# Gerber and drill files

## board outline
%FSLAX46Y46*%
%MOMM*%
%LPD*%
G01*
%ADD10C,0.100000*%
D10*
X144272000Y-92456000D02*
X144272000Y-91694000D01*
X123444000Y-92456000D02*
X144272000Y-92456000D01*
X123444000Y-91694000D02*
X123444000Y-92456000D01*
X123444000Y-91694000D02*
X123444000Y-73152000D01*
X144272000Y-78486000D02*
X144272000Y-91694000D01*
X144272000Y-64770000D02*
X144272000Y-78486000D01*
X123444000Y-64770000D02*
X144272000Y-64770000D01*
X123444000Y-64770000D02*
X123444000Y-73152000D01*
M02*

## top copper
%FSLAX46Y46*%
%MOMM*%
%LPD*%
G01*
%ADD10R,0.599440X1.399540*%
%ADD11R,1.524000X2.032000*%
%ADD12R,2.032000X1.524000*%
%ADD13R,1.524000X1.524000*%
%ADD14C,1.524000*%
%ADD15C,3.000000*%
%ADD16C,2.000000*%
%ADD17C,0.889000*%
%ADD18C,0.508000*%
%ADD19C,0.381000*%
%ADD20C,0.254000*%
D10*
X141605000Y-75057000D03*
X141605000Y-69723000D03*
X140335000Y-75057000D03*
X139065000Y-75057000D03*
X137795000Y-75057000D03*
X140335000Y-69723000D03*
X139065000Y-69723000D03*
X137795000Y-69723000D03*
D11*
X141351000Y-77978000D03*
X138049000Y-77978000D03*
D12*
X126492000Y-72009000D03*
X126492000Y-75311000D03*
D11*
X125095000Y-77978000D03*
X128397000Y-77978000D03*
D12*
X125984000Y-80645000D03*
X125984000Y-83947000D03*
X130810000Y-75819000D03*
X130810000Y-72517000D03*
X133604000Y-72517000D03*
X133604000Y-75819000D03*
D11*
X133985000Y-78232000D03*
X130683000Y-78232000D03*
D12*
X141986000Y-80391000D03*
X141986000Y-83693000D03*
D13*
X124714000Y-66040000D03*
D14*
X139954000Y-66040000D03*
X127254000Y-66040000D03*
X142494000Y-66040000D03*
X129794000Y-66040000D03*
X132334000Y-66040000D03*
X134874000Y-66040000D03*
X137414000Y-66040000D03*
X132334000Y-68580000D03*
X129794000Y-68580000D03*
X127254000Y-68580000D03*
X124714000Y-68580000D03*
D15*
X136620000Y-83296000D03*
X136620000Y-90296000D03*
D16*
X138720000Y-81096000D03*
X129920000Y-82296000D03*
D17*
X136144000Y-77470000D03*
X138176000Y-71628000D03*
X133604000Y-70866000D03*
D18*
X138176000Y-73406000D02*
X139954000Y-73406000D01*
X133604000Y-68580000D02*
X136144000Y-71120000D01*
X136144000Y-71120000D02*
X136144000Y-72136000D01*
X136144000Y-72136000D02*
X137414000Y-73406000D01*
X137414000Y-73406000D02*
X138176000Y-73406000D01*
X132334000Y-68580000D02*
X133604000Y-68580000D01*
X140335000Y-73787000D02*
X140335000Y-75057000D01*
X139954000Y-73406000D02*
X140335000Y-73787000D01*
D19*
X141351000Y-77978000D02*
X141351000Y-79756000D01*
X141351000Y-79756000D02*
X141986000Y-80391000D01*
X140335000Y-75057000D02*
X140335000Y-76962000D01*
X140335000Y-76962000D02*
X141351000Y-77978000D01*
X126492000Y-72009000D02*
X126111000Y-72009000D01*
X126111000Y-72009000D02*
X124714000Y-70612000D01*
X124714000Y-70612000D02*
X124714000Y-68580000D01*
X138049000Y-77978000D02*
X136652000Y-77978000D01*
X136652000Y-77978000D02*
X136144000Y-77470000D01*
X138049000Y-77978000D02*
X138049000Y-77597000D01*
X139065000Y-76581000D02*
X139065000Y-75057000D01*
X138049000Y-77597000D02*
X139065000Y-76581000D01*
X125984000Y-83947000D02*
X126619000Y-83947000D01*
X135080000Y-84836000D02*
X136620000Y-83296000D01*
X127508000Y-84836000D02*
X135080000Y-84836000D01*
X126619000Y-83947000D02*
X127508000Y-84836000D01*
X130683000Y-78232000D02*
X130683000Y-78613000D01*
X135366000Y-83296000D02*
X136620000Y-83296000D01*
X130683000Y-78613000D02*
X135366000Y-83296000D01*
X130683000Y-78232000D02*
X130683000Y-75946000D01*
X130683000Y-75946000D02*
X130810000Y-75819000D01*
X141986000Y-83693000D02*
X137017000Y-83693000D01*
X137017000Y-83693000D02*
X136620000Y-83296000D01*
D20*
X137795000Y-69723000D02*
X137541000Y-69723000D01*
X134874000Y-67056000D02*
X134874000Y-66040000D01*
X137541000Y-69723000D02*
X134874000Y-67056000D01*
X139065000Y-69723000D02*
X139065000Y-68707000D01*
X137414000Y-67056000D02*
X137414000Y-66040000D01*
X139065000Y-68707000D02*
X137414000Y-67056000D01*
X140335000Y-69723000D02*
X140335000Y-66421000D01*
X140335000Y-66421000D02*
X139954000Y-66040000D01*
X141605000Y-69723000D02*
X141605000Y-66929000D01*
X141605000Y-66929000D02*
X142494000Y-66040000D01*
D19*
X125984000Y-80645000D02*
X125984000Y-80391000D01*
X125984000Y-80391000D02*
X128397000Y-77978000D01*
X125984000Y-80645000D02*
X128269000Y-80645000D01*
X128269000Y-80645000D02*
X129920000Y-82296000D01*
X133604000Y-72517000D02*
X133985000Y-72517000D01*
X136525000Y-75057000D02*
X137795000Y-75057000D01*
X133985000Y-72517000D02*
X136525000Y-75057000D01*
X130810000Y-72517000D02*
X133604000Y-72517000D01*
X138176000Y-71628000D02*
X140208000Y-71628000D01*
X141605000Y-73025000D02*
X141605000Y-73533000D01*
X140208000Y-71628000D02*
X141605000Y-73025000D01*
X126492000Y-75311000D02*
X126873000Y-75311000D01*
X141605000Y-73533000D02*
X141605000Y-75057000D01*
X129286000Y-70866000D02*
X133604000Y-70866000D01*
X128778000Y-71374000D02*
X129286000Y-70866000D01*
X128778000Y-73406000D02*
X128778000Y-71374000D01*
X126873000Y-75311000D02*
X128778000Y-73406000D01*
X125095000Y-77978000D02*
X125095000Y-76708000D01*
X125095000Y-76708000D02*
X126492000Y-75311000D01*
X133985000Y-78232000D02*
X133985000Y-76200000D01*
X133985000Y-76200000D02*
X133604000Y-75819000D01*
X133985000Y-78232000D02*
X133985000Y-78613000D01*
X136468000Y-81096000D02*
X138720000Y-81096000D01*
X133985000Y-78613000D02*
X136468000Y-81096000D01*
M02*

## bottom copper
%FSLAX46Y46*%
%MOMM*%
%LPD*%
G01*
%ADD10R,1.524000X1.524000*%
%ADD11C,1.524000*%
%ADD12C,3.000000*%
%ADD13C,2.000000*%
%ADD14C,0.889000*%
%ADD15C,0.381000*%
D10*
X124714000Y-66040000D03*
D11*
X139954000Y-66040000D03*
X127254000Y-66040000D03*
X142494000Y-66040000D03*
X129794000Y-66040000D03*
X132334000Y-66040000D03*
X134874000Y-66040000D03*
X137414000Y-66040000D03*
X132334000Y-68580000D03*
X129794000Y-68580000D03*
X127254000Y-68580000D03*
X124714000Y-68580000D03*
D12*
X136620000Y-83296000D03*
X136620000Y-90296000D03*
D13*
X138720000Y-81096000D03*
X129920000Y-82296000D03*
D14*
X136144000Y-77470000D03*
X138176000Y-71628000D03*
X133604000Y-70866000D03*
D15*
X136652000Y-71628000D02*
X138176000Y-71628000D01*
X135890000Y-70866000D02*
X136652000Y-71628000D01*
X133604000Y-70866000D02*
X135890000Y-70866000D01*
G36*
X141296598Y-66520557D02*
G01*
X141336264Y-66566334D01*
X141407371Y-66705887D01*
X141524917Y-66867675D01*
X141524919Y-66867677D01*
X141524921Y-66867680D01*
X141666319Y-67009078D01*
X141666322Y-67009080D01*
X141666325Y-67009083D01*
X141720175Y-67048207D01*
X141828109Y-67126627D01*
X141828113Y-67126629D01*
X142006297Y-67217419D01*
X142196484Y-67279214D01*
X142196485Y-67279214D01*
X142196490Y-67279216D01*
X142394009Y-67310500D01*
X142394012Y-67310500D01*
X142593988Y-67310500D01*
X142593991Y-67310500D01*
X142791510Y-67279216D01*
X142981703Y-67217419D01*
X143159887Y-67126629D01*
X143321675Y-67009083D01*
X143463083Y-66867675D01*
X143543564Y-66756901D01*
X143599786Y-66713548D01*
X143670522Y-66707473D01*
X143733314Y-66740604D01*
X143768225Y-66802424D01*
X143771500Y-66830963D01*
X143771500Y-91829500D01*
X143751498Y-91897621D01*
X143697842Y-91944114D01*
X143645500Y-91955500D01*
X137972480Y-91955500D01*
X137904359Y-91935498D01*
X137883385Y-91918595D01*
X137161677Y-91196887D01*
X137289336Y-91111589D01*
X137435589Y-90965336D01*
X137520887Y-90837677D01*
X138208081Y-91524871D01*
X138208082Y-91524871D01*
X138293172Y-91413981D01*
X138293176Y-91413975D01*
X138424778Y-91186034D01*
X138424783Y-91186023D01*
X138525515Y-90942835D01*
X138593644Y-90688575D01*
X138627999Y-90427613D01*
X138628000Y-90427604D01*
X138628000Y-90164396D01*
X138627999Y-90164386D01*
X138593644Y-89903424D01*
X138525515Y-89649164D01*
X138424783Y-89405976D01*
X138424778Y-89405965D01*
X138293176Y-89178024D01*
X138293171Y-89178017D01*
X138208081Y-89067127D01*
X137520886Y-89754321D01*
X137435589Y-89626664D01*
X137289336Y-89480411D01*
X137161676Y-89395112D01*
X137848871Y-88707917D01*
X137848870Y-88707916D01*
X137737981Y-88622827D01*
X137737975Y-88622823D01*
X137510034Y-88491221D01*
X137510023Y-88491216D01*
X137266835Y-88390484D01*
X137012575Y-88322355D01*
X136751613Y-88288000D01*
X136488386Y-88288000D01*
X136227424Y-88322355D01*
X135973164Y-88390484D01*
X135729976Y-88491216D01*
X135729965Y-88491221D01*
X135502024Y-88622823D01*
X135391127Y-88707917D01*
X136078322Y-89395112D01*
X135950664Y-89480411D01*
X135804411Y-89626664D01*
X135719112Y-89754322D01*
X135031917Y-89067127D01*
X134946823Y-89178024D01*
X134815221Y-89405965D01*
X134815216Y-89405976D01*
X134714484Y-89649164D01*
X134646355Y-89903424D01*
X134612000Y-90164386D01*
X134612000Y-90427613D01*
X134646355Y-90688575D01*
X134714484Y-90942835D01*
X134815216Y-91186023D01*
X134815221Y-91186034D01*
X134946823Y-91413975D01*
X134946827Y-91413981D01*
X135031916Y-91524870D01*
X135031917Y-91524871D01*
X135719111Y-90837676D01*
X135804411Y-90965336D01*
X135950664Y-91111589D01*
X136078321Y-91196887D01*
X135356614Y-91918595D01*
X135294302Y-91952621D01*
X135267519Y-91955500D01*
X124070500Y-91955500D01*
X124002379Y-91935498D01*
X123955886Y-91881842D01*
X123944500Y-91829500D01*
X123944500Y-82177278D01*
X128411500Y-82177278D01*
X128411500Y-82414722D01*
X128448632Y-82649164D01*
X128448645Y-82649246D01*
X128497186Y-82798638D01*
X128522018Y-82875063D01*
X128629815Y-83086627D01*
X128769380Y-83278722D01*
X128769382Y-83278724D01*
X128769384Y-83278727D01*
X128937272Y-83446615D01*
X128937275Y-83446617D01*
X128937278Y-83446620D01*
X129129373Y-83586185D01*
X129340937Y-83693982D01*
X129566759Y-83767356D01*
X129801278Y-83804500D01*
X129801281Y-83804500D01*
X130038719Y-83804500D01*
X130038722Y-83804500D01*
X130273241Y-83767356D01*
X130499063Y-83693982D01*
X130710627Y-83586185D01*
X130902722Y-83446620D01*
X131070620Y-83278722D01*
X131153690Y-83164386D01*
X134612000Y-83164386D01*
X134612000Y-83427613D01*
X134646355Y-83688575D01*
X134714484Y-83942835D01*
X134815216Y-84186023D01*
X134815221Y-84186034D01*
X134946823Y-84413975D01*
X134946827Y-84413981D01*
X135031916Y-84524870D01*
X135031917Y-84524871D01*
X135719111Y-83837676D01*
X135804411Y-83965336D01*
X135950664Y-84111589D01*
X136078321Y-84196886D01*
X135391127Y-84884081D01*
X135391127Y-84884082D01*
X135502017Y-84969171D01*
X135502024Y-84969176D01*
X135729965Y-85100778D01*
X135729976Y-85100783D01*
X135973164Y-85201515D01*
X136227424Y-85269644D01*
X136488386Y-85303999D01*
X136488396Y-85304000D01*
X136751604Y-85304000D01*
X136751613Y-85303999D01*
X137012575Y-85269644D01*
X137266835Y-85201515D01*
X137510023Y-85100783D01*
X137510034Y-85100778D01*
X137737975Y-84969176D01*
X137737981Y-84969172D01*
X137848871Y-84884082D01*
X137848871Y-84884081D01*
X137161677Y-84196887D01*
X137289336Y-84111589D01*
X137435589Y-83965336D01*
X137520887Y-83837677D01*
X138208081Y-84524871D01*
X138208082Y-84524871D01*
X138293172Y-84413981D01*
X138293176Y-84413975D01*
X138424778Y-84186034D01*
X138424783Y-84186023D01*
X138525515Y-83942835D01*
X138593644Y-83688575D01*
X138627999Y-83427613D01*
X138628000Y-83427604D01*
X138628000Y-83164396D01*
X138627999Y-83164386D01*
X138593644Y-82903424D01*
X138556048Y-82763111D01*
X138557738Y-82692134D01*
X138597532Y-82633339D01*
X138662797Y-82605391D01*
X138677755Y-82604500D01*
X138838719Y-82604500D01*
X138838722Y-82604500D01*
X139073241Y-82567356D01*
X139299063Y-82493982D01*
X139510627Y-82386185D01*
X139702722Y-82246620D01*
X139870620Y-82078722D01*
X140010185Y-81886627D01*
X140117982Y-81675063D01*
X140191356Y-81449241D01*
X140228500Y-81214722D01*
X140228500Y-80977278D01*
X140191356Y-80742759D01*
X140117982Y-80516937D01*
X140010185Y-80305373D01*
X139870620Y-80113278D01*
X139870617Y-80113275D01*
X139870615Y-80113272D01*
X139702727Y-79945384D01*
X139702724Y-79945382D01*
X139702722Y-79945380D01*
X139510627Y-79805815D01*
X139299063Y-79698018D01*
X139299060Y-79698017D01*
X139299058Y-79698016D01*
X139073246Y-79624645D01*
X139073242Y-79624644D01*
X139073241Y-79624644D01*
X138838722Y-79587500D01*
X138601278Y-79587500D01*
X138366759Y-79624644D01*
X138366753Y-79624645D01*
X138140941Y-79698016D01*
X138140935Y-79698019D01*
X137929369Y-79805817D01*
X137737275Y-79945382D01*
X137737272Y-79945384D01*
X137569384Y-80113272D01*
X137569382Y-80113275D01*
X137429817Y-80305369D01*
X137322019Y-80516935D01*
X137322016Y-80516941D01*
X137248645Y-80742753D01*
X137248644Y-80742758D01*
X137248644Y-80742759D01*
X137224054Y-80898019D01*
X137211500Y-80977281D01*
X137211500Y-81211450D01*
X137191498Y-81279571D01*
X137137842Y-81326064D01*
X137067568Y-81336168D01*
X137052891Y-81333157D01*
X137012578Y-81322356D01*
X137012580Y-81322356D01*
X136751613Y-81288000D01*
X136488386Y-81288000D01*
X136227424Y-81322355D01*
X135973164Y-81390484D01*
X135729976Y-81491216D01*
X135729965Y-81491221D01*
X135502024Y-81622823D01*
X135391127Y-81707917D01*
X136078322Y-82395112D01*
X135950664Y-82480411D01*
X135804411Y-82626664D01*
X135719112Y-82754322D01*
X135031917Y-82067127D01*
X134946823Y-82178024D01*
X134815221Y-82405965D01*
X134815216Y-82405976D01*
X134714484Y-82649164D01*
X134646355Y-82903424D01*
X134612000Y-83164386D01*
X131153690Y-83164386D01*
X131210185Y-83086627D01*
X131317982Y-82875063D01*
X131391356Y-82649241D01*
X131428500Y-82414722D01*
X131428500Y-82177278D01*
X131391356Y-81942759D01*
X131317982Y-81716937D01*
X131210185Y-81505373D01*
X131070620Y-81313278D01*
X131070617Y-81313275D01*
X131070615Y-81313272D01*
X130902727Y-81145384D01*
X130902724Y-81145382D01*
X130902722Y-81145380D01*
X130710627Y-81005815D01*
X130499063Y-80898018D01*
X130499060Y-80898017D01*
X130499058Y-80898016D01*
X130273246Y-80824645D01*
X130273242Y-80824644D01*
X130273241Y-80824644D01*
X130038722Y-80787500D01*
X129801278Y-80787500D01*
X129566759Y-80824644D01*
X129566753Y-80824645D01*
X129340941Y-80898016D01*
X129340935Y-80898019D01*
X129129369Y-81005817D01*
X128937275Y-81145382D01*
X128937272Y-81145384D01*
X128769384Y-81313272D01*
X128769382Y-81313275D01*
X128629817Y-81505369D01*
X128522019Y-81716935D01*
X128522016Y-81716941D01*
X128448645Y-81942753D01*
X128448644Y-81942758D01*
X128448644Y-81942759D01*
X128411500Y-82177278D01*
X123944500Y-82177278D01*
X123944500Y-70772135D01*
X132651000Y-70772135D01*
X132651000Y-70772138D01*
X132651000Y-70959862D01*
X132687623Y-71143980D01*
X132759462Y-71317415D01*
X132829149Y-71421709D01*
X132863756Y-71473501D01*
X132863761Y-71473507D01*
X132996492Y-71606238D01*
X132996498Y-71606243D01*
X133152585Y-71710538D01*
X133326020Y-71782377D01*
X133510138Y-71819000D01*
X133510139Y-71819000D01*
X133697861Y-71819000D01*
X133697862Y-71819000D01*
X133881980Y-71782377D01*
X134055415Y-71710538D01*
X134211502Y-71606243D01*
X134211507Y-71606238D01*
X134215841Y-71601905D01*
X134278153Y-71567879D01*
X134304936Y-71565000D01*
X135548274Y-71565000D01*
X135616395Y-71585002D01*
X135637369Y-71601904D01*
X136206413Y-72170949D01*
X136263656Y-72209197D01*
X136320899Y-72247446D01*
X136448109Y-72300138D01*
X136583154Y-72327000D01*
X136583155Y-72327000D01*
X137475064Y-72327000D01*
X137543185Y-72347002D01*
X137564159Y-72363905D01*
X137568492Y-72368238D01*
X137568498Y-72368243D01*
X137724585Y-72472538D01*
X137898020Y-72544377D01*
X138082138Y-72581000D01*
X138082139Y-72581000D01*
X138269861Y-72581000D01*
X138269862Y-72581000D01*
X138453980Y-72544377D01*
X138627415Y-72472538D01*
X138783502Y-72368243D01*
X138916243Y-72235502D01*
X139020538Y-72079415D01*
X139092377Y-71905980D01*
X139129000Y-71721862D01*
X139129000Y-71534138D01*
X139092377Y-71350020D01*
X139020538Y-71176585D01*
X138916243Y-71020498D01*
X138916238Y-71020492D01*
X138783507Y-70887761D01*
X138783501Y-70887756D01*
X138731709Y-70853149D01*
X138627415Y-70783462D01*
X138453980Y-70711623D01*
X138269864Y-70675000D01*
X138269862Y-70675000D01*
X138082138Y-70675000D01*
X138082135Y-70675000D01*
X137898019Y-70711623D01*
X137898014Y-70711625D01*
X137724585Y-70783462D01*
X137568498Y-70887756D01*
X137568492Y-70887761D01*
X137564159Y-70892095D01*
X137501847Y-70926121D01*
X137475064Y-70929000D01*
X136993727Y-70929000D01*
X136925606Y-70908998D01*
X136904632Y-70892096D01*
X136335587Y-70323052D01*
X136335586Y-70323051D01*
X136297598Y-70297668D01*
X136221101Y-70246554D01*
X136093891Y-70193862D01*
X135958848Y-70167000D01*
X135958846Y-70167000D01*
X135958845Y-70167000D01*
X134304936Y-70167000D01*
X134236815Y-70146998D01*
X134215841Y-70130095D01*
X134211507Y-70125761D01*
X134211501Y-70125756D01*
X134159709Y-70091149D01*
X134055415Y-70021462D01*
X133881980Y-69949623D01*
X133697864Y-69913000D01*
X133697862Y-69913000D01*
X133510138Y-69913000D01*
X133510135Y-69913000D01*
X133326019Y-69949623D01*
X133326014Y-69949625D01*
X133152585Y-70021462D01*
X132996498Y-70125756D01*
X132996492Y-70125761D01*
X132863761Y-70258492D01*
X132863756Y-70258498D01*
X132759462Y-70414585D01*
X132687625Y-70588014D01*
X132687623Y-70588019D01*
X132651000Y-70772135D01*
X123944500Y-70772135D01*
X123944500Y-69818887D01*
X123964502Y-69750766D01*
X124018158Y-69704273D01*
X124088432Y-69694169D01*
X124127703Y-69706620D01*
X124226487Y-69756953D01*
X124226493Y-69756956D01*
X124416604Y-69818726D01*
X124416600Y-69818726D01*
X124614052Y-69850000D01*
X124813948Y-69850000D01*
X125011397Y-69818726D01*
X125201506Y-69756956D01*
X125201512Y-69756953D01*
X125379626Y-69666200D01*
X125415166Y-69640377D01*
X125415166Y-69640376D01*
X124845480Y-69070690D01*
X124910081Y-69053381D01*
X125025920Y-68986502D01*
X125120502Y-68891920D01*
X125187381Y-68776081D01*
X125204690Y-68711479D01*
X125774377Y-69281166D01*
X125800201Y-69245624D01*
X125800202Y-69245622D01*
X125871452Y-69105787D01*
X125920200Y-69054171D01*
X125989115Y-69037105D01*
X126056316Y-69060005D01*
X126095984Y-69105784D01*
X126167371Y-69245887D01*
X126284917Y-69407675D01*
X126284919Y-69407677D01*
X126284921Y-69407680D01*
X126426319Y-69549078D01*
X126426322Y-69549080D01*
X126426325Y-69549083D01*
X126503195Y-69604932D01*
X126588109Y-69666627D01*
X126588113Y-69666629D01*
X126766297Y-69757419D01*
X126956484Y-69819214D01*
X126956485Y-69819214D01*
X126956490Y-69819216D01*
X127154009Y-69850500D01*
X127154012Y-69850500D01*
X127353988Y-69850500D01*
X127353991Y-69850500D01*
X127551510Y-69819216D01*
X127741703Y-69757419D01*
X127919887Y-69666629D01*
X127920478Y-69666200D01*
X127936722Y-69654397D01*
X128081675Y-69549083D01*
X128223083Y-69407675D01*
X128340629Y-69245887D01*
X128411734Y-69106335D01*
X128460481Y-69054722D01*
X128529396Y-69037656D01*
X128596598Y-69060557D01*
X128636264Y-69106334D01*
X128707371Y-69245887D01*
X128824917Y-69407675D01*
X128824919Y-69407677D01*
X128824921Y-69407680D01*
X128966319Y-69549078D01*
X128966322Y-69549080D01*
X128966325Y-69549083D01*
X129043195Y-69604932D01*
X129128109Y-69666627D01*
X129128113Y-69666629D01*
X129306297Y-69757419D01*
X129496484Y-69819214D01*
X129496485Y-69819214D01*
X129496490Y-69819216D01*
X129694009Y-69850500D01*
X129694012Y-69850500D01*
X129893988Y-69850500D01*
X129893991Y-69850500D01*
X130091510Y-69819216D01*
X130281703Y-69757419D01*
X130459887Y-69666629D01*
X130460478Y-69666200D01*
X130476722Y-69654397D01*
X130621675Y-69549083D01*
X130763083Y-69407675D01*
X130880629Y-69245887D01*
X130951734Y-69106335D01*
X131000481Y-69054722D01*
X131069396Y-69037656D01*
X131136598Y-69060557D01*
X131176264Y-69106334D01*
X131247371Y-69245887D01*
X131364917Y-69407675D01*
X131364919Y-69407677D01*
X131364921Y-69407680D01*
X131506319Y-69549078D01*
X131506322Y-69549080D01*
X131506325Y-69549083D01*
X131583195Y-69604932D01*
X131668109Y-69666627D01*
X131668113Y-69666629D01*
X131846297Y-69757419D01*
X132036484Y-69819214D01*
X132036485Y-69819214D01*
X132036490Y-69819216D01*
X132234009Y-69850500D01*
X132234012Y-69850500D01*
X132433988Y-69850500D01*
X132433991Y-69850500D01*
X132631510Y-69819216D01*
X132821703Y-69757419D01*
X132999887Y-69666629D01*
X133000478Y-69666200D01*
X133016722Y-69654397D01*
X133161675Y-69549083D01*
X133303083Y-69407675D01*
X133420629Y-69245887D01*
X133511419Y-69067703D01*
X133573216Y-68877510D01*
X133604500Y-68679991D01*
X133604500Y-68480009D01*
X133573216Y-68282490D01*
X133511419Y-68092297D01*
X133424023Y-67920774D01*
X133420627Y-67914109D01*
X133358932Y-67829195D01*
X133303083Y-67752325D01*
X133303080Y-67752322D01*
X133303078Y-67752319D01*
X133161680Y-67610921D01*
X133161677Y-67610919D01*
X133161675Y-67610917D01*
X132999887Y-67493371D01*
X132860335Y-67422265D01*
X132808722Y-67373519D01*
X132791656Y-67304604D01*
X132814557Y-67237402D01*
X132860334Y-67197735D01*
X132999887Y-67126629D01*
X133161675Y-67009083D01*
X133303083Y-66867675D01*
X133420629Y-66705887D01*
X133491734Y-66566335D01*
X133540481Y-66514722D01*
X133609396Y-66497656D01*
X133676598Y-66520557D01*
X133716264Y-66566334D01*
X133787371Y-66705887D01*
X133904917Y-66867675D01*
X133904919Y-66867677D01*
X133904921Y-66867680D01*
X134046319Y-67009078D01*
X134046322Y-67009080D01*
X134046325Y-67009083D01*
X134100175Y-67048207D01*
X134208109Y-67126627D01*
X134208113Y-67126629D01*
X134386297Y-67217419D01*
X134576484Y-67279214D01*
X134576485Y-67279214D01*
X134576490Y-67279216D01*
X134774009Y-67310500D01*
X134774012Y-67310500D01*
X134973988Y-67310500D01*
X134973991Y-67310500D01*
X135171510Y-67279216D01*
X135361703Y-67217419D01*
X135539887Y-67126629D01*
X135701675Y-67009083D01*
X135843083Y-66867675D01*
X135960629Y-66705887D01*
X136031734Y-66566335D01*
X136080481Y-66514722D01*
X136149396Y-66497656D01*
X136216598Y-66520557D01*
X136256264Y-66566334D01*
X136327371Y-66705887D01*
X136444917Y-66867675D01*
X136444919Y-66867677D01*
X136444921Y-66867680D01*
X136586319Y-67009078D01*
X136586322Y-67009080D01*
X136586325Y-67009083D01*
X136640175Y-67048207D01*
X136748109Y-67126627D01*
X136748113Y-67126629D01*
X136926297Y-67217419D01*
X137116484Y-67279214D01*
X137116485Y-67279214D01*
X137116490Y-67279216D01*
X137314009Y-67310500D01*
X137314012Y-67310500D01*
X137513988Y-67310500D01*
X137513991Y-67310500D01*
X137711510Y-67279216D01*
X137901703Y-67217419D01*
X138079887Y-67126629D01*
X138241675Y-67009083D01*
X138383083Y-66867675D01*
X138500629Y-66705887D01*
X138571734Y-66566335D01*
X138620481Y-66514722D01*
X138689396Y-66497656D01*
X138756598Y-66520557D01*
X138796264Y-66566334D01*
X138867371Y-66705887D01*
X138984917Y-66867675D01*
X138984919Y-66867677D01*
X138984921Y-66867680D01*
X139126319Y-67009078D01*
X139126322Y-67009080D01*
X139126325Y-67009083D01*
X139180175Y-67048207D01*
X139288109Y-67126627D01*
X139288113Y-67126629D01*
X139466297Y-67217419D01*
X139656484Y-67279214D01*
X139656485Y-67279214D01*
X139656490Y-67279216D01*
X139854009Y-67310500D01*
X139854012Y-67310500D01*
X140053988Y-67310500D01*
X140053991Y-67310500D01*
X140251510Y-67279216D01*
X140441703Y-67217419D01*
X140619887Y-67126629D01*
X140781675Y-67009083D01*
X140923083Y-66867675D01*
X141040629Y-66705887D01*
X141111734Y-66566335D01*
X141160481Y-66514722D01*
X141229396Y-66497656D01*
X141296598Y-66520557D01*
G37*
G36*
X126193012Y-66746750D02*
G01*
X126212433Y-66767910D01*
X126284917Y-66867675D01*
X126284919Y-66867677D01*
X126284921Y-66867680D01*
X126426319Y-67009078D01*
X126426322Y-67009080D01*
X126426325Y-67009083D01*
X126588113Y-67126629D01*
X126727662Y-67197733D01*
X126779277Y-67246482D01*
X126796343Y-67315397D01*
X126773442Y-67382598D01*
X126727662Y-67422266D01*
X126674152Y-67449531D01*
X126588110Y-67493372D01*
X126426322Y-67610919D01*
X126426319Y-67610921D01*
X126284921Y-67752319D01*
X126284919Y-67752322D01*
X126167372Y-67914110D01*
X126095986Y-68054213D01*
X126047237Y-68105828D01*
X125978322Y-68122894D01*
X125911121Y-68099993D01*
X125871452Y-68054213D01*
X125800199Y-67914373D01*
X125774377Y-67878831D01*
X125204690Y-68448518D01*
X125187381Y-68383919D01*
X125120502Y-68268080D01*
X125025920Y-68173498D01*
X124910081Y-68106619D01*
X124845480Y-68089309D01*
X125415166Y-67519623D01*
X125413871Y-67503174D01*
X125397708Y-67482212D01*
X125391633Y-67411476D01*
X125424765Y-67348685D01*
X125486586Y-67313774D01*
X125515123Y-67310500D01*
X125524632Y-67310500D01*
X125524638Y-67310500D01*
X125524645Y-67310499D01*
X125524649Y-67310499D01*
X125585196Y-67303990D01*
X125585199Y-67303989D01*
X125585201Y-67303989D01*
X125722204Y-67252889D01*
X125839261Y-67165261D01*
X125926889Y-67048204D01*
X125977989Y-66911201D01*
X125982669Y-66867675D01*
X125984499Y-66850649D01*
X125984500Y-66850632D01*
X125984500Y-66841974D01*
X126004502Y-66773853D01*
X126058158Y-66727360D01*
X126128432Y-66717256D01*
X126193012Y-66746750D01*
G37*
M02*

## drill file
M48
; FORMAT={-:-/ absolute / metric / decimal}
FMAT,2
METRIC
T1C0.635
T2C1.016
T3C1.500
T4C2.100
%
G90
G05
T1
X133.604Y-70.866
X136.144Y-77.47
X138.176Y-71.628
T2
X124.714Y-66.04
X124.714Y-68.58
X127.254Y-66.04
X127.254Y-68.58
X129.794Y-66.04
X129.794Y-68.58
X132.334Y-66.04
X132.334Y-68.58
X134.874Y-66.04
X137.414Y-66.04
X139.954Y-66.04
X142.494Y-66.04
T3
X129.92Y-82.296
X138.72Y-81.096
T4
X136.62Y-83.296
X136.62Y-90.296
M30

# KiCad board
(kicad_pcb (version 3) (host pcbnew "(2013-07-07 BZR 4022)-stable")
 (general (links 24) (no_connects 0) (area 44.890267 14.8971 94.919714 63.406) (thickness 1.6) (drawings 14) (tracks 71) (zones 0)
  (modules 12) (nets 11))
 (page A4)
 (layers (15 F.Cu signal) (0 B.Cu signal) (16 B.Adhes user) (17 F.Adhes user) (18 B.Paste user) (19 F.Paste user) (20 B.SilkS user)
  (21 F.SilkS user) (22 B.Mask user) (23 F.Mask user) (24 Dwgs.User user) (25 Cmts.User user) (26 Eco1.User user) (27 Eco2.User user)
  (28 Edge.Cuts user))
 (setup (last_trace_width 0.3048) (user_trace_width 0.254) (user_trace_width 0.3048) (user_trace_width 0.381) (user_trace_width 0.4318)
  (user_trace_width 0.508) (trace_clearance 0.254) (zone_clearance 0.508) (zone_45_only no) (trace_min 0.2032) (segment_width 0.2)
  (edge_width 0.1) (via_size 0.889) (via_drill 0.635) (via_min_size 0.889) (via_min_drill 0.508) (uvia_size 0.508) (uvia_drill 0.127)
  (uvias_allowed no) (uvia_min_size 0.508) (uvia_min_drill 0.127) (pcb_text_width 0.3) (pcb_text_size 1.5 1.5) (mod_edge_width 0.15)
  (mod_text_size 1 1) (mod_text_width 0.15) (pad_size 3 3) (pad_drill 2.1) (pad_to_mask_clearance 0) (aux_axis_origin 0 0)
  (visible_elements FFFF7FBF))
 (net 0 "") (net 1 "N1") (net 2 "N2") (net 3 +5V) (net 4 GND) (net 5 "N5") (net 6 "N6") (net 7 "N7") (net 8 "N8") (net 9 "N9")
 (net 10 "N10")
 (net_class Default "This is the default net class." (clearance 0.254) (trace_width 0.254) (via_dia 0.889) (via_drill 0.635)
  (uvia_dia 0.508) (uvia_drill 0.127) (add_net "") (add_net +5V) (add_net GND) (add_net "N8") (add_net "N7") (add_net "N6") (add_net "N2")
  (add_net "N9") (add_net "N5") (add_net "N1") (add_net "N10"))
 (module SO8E (layer F.Cu) (at 139.7 72.39 180)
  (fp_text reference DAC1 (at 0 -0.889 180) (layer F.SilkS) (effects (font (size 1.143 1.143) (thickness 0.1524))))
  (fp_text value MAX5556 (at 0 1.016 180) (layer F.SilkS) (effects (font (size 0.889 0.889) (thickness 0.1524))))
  (pad 8 smd rect (at -1.905 -2.667 180) (size 0.59944 1.39954) (layers F.Cu F.Paste F.Mask) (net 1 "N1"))
  (pad 1 smd rect (at -1.905 2.667 180) (size 0.59944 1.39954) (layers F.Cu F.Paste F.Mask) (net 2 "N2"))
  (pad 7 smd rect (at -0.635 -2.667 180) (size 0.59944 1.39954) (layers F.Cu F.Paste F.Mask) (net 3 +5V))
  (pad 6 smd rect (at 0.635 -2.667 180) (size 0.59944 1.39954) (layers F.Cu F.Paste F.Mask) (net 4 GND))
  (pad 5 smd rect (at 1.905 -2.667 180) (size 0.59944 1.39954) (layers F.Cu F.Paste F.Mask) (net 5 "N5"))
  (pad 2 smd rect (at -0.635 2.667 180) (size 0.59944 1.39954) (layers F.Cu F.Paste F.Mask) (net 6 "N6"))
  (pad 3 smd rect (at 0.635 2.667 180) (size 0.59944 1.39954) (layers F.Cu F.Paste F.Mask) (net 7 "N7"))
  (pad 4 smd rect (at 1.905 2.667 180) (size 0.59944 1.39954) (layers F.Cu F.Paste F.Mask) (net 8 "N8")))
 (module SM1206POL (layer F.Cu) (at 139.7 77.978 180)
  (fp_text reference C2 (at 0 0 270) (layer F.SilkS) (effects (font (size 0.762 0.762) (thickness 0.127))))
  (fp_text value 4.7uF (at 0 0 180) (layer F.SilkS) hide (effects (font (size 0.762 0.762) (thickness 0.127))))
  (pad 1 smd rect (at -1.651 0 180) (size 1.524 2.032) (layers F.Cu F.Paste F.Mask) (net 3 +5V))
  (pad 2 smd rect (at 1.651 0 180) (size 1.524 2.032) (layers F.Cu F.Paste F.Mask) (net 4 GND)))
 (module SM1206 (layer F.Cu) (at 126.492 73.66 270)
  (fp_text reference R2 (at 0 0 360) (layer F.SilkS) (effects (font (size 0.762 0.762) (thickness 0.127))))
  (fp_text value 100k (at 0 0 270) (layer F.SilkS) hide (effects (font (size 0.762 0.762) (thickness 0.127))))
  (pad 1 smd rect (at -1.651 0 270) (size 1.524 2.032) (layers F.Cu F.Paste F.Mask) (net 4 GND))
  (pad 2 smd rect (at 1.651 0 270) (size 1.524 2.032) (layers F.Cu F.Paste F.Mask) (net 1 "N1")))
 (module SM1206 (layer F.Cu) (at 126.746 77.978)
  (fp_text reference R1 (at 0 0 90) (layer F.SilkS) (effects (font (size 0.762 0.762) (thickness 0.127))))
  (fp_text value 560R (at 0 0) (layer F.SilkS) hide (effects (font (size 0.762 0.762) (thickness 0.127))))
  (pad 1 smd rect (at -1.651 0) (size 1.524 2.032) (layers F.Cu F.Paste F.Mask) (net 1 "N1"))
  (pad 2 smd rect (at 1.651 0) (size 1.524 2.032) (layers F.Cu F.Paste F.Mask) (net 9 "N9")))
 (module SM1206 (layer F.Cu) (at 125.984 82.296 270)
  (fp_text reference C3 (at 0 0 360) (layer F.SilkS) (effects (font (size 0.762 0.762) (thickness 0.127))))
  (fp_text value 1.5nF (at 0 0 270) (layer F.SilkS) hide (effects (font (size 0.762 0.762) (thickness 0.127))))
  (pad 1 smd rect (at -1.651 0 270) (size 1.524 2.032) (layers F.Cu F.Paste F.Mask) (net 9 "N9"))
  (pad 2 smd rect (at 1.651 0 270) (size 1.524 2.032) (layers F.Cu F.Paste F.Mask) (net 4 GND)))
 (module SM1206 (layer F.Cu) (at 130.81 74.168 90)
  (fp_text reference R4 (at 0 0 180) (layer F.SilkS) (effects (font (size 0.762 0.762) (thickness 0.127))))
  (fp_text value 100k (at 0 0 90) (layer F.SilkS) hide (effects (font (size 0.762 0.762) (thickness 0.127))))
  (pad 1 smd rect (at -1.651 0 90) (size 1.524 2.032) (layers F.Cu F.Paste F.Mask) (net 4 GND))
  (pad 2 smd rect (at 1.651 0 90) (size 1.524 2.032) (layers F.Cu F.Paste F.Mask) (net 5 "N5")))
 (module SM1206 (layer F.Cu) (at 133.604 74.168 270)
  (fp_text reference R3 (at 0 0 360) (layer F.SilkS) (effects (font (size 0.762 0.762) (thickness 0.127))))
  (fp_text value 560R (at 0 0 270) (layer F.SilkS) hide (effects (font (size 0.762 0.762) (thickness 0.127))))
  (pad 1 smd rect (at -1.651 0 270) (size 1.524 2.032) (layers F.Cu F.Paste F.Mask) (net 5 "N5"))
  (pad 2 smd rect (at 1.651 0 270) (size 1.524 2.032) (layers F.Cu F.Paste F.Mask) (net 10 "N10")))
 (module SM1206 (layer F.Cu) (at 132.334 78.232 180)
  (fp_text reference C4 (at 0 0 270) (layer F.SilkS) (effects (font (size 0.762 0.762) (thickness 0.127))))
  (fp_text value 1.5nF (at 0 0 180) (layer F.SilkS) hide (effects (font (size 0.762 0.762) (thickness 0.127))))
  (pad 1 smd rect (at -1.651 0 180) (size 1.524 2.032) (layers F.Cu F.Paste F.Mask) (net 10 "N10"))
  (pad 2 smd rect (at 1.651 0 180) (size 1.524 2.032) (layers F.Cu F.Paste F.Mask) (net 4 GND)))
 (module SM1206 (layer F.Cu) (at 141.986 82.042 270)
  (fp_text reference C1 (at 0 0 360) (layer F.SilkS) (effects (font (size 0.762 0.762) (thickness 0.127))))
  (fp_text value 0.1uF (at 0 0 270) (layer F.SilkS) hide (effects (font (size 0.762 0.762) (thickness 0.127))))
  (pad 1 smd rect (at -1.651 0 270) (size 1.524 2.032) (layers F.Cu F.Paste F.Mask) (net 3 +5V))
  (pad 2 smd rect (at 1.651 0 270) (size 1.524 2.032) (layers F.Cu F.Paste F.Mask) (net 4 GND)))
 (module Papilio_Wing (layer F.Cu) (at 134.112 67.564)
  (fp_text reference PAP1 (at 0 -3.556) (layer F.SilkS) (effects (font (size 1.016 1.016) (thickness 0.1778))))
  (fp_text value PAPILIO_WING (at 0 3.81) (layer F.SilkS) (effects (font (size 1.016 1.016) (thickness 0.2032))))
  (pad 1 thru_hole rect (at -9.398 -1.524) (size 1.524 1.524) (drill 1.016) (layers *.Cu *.Mask F.SilkS))
  (pad 7 thru_hole circle (at 5.842 -1.524) (size 1.524 1.524) (drill 1.016) (layers *.Cu *.Mask F.SilkS) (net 6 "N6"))
  (pad 2 thru_hole circle (at -6.858 -1.524) (size 1.524 1.524) (drill 1.016) (layers *.Cu *.Mask F.SilkS))
  (pad 8 thru_hole circle (at 8.382 -1.524) (size 1.524 1.524) (drill 1.016) (layers *.Cu *.Mask F.SilkS) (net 2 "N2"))
  (pad 3 thru_hole circle (at -4.318 -1.524) (size 1.524 1.524) (drill 1.016) (layers *.Cu *.Mask F.SilkS))
  (pad 4 thru_hole circle (at -1.778 -1.524) (size 1.524 1.524) (drill 1.016) (layers *.Cu *.Mask F.SilkS))
  (pad 5 thru_hole circle (at 0.762 -1.524) (size 1.524 1.524) (drill 1.016) (layers *.Cu *.Mask F.SilkS) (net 8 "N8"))
  (pad 6 thru_hole circle (at 3.302 -1.524) (size 1.524 1.524) (drill 1.016) (layers *.Cu *.Mask F.SilkS) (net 7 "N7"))
  (pad 9 thru_hole circle (at -1.778 1.016) (size 1.524 1.524) (drill 1.016) (layers *.Cu *.Mask F.SilkS) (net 3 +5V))
  (pad 10 thru_hole circle (at -4.318 1.016) (size 1.524 1.524) (drill 1.016) (layers *.Cu *.Mask F.SilkS))
  (pad 11 thru_hole circle (at -6.858 1.016) (size 1.524 1.524) (drill 1.016) (layers *.Cu *.Mask F.SilkS))
  (pad 12 thru_hole circle (at -9.398 1.016) (size 1.524 1.524) (drill 1.016) (layers *.Cu *.Mask F.SilkS) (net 4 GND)))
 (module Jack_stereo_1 (layer F.Cu) (at 134.62 82.296)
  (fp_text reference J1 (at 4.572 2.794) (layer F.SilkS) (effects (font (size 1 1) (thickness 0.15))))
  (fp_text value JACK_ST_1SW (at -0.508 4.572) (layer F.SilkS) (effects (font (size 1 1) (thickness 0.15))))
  (pad 1 thru_hole circle (at 2 1) (size 3 3) (drill 2.1) (layers *.Cu *.Mask F.SilkS) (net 4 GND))
  (pad 4 thru_hole circle (at 2 8) (size 3 3) (drill 2.1) (layers *.Cu *.Mask F.SilkS) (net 4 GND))
  (pad 3 thru_hole circle (at 4.1 -1.2) (size 2 2) (drill 1.5) (layers *.Cu *.Mask F.SilkS) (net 10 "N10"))
  (pad 2 thru_hole circle (at -4.7 0) (size 2 2) (drill 1.5) (layers *.Cu *.Mask F.SilkS) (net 9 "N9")))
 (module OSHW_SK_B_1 (layer F.Cu) (at 129.794 76.708)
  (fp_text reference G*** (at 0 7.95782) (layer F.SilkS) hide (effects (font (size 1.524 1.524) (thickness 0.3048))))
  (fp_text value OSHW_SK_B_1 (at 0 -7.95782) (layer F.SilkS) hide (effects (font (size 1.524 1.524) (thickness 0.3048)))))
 (gr_line (start 144.272 92.456) (end 144.272 91.694) (angle 90) (layer Edge.Cuts) (width 0.1))
 (gr_line (start 123.444 92.456) (end 144.272 92.456) (angle 90) (layer Edge.Cuts) (width 0.1))
 (gr_line (start 123.444 91.694) (end 123.444 92.456) (angle 90) (layer Edge.Cuts) (width 0.1))
 (gr_line (start 123.444 91.694) (end 123.444 73.152) (angle 90) (layer Edge.Cuts) (width 0.1))
 (gr_line (start 144.272 78.486) (end 144.272 91.694) (angle 90) (layer Edge.Cuts) (width 0.1))
 (gr_line (start 144.272 64.77) (end 144.272 78.486) (angle 90) (layer Edge.Cuts) (width 0.1))
 (gr_line (start 123.444 64.77) (end 144.272 64.77) (angle 90) (layer Edge.Cuts) (width 0.1))
 (gr_line (start 123.444 64.77) (end 123.444 73.152) (angle 90) (layer Edge.Cuts) (width 0.1))
 (segment (start 138.176 73.406) (end 139.954 73.406) (width 0.508) (layer F.Cu) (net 3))
 (segment (start 133.604 68.58) (end 136.144 71.12) (width 0.508) (layer F.Cu) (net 3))
 (segment (start 136.144 71.12) (end 136.144 72.136) (width 0.508) (layer F.Cu) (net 3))
 (segment (start 136.144 72.136) (end 137.414 73.406) (width 0.508) (layer F.Cu) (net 3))
 (segment (start 137.414 73.406) (end 138.176 73.406) (width 0.508) (layer F.Cu) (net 3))
 (segment (start 132.334 68.58) (end 133.604 68.58) (width 0.508) (layer F.Cu) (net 3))
 (segment (start 140.335 73.787) (end 140.335 75.057) (width 0.508) (layer F.Cu) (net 3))
 (segment (start 139.954 73.406) (end 140.335 73.787) (width 0.508) (layer F.Cu) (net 3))
 (segment (start 141.351 77.978) (end 141.351 79.756) (width 0.381) (layer F.Cu) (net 3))
 (segment (start 141.351 79.756) (end 141.986 80.391) (width 0.381) (layer F.Cu) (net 3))
 (segment (start 140.335 75.057) (end 140.335 76.962) (width 0.381) (layer F.Cu) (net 3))
 (segment (start 140.335 76.962) (end 141.351 77.978) (width 0.381) (layer F.Cu) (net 3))
 (segment (start 126.492 72.009) (end 126.111 72.009) (width 0.381) (layer F.Cu) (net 4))
 (segment (start 126.111 72.009) (end 124.714 70.612) (width 0.381) (layer F.Cu) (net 4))
 (segment (start 124.714 70.612) (end 124.714 68.58) (width 0.381) (layer F.Cu) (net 4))
 (segment (start 138.049 77.978) (end 136.652 77.978) (width 0.381) (layer F.Cu) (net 4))
 (via (at 136.144 77.47) (size 0.889) (layers F.Cu B.Cu) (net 4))
 (segment (start 136.652 77.978) (end 136.144 77.47) (width 0.381) (layer F.Cu) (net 4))
 (segment (start 138.049 77.978) (end 138.049 77.597) (width 0.381) (layer F.Cu) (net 4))
 (segment (start 139.065 76.581) (end 139.065 75.057) (width 0.381) (layer F.Cu) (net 4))
 (segment (start 138.049 77.597) (end 139.065 76.581) (width 0.381) (layer F.Cu) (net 4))
 (segment (start 125.984 83.947) (end 126.619 83.947) (width 0.381) (layer F.Cu) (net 4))
 (segment (start 135.08 84.836) (end 136.62 83.296) (width 0.381) (layer F.Cu) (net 4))
 (segment (start 127.508 84.836) (end 135.08 84.836) (width 0.381) (layer F.Cu) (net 4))
 (segment (start 126.619 83.947) (end 127.508 84.836) (width 0.381) (layer F.Cu) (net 4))
 (segment (start 130.683 78.232) (end 130.683 78.613) (width 0.381) (layer F.Cu) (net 4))
 (segment (start 135.366 83.296) (end 136.62 83.296) (width 0.381) (layer F.Cu) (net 4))
 (segment (start 130.683 78.613) (end 135.366 83.296) (width 0.381) (layer F.Cu) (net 4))
 (segment (start 130.683 78.232) (end 130.683 75.946) (width 0.381) (layer F.Cu) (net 4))
 (segment (start 130.683 75.946) (end 130.81 75.819) (width 0.381) (layer F.Cu) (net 4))
 (segment (start 141.986 83.693) (end 137.017 83.693) (width 0.381) (layer F.Cu) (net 4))
 (segment (start 137.017 83.693) (end 136.62 83.296) (width 0.381) (layer F.Cu) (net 4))
 (segment (start 137.795 69.723) (end 137.541 69.723) (width 0.254) (layer F.Cu) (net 8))
 (segment (start 134.874 67.056) (end 134.874 66.04) (width 0.254) (layer F.Cu) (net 8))
 (segment (start 137.541 69.723) (end 134.874 67.056) (width 0.254) (layer F.Cu) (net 8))
 (segment (start 139.065 69.723) (end 139.065 68.707) (width 0.254) (layer F.Cu) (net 7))
 (segment (start 137.414 67.056) (end 137.414 66.04) (width 0.254) (layer F.Cu) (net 7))
 (segment (start 139.065 68.707) (end 137.414 67.056) (width 0.254) (layer F.Cu) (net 7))
 (segment (start 140.335 69.723) (end 140.335 66.421) (width 0.254) (layer F.Cu) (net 6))
 (segment (start 140.335 66.421) (end 139.954 66.04) (width 0.254) (layer F.Cu) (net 6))
 (segment (start 141.605 69.723) (end 141.605 66.929) (width 0.254) (layer F.Cu) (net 2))
 (segment (start 141.605 66.929) (end 142.494 66.04) (width 0.254) (layer F.Cu) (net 2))
 (segment (start 125.984 80.645) (end 125.984 80.391) (width 0.381) (layer F.Cu) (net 9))
 (segment (start 125.984 80.391) (end 128.397 77.978) (width 0.381) (layer F.Cu) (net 9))
 (segment (start 125.984 80.645) (end 128.269 80.645) (width 0.381) (layer F.Cu) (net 9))
 (segment (start 128.269 80.645) (end 129.92 82.296) (width 0.381) (layer F.Cu) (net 9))
 (segment (start 133.604 72.517) (end 133.985 72.517) (width 0.381) (layer F.Cu) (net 5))
 (segment (start 136.525 75.057) (end 137.795 75.057) (width 0.381) (layer F.Cu) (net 5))
 (segment (start 133.985 72.517) (end 136.525 75.057) (width 0.381) (layer F.Cu) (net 5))
 (segment (start 130.81 72.517) (end 133.604 72.517) (width 0.381) (layer F.Cu) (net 5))
 (segment (start 138.176 71.628) (end 140.208 71.628) (width 0.381) (layer F.Cu) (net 1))
 (segment (start 141.605 73.025) (end 141.605 73.533) (width 0.381) (layer F.Cu) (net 1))
 (segment (start 140.208 71.628) (end 141.605 73.025) (width 0.381) (layer F.Cu) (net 1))
 (segment (start 126.492 75.311) (end 126.873 75.311) (width 0.381) (layer F.Cu) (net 1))
 (segment (start 141.605 73.533) (end 141.605 75.057) (width 0.381) (layer F.Cu) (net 1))
 (via (at 138.176 71.628) (size 0.889) (layers F.Cu B.Cu) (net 1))
 (segment (start 136.652 71.628) (end 138.176 71.628) (width 0.381) (layer B.Cu) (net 1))
 (segment (start 135.89 70.866) (end 136.652 71.628) (width 0.381) (layer B.Cu) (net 1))
 (segment (start 133.604 70.866) (end 135.89 70.866) (width 0.381) (layer B.Cu) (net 1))
 (via (at 133.604 70.866) (size 0.889) (layers F.Cu B.Cu) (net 1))
 (segment (start 129.286 70.866) (end 133.604 70.866) (width 0.381) (layer F.Cu) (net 1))
 (segment (start 128.778 71.374) (end 129.286 70.866) (width 0.381) (layer F.Cu) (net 1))
 (segment (start 128.778 73.406) (end 128.778 71.374) (width 0.381) (layer F.Cu) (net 1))
 (segment (start 126.873 75.311) (end 128.778 73.406) (width 0.381) (layer F.Cu) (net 1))
 (segment (start 125.095 77.978) (end 125.095 76.708) (width 0.381) (layer F.Cu) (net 1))
 (segment (start 125.095 76.708) (end 126.492 75.311) (width 0.381) (layer F.Cu) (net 1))
 (segment (start 133.985 78.232) (end 133.985 76.2) (width 0.381) (layer F.Cu) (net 10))
 (segment (start 133.985 76.2) (end 133.604 75.819) (width 0.381) (layer F.Cu) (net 10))
 (segment (start 133.985 78.232) (end 133.985 78.613) (width 0.381) (layer F.Cu) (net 10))
 (segment (start 136.468 81.096) (end 138.72 81.096) (width 0.381) (layer F.Cu) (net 10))
 (segment (start 133.985 78.613) (end 136.468 81.096) (width 0.381) (layer F.Cu) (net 10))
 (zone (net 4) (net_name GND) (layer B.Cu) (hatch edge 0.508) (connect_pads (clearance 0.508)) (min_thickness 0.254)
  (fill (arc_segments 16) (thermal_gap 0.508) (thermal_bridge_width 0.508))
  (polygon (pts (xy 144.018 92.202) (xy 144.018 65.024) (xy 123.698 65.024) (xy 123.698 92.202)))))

